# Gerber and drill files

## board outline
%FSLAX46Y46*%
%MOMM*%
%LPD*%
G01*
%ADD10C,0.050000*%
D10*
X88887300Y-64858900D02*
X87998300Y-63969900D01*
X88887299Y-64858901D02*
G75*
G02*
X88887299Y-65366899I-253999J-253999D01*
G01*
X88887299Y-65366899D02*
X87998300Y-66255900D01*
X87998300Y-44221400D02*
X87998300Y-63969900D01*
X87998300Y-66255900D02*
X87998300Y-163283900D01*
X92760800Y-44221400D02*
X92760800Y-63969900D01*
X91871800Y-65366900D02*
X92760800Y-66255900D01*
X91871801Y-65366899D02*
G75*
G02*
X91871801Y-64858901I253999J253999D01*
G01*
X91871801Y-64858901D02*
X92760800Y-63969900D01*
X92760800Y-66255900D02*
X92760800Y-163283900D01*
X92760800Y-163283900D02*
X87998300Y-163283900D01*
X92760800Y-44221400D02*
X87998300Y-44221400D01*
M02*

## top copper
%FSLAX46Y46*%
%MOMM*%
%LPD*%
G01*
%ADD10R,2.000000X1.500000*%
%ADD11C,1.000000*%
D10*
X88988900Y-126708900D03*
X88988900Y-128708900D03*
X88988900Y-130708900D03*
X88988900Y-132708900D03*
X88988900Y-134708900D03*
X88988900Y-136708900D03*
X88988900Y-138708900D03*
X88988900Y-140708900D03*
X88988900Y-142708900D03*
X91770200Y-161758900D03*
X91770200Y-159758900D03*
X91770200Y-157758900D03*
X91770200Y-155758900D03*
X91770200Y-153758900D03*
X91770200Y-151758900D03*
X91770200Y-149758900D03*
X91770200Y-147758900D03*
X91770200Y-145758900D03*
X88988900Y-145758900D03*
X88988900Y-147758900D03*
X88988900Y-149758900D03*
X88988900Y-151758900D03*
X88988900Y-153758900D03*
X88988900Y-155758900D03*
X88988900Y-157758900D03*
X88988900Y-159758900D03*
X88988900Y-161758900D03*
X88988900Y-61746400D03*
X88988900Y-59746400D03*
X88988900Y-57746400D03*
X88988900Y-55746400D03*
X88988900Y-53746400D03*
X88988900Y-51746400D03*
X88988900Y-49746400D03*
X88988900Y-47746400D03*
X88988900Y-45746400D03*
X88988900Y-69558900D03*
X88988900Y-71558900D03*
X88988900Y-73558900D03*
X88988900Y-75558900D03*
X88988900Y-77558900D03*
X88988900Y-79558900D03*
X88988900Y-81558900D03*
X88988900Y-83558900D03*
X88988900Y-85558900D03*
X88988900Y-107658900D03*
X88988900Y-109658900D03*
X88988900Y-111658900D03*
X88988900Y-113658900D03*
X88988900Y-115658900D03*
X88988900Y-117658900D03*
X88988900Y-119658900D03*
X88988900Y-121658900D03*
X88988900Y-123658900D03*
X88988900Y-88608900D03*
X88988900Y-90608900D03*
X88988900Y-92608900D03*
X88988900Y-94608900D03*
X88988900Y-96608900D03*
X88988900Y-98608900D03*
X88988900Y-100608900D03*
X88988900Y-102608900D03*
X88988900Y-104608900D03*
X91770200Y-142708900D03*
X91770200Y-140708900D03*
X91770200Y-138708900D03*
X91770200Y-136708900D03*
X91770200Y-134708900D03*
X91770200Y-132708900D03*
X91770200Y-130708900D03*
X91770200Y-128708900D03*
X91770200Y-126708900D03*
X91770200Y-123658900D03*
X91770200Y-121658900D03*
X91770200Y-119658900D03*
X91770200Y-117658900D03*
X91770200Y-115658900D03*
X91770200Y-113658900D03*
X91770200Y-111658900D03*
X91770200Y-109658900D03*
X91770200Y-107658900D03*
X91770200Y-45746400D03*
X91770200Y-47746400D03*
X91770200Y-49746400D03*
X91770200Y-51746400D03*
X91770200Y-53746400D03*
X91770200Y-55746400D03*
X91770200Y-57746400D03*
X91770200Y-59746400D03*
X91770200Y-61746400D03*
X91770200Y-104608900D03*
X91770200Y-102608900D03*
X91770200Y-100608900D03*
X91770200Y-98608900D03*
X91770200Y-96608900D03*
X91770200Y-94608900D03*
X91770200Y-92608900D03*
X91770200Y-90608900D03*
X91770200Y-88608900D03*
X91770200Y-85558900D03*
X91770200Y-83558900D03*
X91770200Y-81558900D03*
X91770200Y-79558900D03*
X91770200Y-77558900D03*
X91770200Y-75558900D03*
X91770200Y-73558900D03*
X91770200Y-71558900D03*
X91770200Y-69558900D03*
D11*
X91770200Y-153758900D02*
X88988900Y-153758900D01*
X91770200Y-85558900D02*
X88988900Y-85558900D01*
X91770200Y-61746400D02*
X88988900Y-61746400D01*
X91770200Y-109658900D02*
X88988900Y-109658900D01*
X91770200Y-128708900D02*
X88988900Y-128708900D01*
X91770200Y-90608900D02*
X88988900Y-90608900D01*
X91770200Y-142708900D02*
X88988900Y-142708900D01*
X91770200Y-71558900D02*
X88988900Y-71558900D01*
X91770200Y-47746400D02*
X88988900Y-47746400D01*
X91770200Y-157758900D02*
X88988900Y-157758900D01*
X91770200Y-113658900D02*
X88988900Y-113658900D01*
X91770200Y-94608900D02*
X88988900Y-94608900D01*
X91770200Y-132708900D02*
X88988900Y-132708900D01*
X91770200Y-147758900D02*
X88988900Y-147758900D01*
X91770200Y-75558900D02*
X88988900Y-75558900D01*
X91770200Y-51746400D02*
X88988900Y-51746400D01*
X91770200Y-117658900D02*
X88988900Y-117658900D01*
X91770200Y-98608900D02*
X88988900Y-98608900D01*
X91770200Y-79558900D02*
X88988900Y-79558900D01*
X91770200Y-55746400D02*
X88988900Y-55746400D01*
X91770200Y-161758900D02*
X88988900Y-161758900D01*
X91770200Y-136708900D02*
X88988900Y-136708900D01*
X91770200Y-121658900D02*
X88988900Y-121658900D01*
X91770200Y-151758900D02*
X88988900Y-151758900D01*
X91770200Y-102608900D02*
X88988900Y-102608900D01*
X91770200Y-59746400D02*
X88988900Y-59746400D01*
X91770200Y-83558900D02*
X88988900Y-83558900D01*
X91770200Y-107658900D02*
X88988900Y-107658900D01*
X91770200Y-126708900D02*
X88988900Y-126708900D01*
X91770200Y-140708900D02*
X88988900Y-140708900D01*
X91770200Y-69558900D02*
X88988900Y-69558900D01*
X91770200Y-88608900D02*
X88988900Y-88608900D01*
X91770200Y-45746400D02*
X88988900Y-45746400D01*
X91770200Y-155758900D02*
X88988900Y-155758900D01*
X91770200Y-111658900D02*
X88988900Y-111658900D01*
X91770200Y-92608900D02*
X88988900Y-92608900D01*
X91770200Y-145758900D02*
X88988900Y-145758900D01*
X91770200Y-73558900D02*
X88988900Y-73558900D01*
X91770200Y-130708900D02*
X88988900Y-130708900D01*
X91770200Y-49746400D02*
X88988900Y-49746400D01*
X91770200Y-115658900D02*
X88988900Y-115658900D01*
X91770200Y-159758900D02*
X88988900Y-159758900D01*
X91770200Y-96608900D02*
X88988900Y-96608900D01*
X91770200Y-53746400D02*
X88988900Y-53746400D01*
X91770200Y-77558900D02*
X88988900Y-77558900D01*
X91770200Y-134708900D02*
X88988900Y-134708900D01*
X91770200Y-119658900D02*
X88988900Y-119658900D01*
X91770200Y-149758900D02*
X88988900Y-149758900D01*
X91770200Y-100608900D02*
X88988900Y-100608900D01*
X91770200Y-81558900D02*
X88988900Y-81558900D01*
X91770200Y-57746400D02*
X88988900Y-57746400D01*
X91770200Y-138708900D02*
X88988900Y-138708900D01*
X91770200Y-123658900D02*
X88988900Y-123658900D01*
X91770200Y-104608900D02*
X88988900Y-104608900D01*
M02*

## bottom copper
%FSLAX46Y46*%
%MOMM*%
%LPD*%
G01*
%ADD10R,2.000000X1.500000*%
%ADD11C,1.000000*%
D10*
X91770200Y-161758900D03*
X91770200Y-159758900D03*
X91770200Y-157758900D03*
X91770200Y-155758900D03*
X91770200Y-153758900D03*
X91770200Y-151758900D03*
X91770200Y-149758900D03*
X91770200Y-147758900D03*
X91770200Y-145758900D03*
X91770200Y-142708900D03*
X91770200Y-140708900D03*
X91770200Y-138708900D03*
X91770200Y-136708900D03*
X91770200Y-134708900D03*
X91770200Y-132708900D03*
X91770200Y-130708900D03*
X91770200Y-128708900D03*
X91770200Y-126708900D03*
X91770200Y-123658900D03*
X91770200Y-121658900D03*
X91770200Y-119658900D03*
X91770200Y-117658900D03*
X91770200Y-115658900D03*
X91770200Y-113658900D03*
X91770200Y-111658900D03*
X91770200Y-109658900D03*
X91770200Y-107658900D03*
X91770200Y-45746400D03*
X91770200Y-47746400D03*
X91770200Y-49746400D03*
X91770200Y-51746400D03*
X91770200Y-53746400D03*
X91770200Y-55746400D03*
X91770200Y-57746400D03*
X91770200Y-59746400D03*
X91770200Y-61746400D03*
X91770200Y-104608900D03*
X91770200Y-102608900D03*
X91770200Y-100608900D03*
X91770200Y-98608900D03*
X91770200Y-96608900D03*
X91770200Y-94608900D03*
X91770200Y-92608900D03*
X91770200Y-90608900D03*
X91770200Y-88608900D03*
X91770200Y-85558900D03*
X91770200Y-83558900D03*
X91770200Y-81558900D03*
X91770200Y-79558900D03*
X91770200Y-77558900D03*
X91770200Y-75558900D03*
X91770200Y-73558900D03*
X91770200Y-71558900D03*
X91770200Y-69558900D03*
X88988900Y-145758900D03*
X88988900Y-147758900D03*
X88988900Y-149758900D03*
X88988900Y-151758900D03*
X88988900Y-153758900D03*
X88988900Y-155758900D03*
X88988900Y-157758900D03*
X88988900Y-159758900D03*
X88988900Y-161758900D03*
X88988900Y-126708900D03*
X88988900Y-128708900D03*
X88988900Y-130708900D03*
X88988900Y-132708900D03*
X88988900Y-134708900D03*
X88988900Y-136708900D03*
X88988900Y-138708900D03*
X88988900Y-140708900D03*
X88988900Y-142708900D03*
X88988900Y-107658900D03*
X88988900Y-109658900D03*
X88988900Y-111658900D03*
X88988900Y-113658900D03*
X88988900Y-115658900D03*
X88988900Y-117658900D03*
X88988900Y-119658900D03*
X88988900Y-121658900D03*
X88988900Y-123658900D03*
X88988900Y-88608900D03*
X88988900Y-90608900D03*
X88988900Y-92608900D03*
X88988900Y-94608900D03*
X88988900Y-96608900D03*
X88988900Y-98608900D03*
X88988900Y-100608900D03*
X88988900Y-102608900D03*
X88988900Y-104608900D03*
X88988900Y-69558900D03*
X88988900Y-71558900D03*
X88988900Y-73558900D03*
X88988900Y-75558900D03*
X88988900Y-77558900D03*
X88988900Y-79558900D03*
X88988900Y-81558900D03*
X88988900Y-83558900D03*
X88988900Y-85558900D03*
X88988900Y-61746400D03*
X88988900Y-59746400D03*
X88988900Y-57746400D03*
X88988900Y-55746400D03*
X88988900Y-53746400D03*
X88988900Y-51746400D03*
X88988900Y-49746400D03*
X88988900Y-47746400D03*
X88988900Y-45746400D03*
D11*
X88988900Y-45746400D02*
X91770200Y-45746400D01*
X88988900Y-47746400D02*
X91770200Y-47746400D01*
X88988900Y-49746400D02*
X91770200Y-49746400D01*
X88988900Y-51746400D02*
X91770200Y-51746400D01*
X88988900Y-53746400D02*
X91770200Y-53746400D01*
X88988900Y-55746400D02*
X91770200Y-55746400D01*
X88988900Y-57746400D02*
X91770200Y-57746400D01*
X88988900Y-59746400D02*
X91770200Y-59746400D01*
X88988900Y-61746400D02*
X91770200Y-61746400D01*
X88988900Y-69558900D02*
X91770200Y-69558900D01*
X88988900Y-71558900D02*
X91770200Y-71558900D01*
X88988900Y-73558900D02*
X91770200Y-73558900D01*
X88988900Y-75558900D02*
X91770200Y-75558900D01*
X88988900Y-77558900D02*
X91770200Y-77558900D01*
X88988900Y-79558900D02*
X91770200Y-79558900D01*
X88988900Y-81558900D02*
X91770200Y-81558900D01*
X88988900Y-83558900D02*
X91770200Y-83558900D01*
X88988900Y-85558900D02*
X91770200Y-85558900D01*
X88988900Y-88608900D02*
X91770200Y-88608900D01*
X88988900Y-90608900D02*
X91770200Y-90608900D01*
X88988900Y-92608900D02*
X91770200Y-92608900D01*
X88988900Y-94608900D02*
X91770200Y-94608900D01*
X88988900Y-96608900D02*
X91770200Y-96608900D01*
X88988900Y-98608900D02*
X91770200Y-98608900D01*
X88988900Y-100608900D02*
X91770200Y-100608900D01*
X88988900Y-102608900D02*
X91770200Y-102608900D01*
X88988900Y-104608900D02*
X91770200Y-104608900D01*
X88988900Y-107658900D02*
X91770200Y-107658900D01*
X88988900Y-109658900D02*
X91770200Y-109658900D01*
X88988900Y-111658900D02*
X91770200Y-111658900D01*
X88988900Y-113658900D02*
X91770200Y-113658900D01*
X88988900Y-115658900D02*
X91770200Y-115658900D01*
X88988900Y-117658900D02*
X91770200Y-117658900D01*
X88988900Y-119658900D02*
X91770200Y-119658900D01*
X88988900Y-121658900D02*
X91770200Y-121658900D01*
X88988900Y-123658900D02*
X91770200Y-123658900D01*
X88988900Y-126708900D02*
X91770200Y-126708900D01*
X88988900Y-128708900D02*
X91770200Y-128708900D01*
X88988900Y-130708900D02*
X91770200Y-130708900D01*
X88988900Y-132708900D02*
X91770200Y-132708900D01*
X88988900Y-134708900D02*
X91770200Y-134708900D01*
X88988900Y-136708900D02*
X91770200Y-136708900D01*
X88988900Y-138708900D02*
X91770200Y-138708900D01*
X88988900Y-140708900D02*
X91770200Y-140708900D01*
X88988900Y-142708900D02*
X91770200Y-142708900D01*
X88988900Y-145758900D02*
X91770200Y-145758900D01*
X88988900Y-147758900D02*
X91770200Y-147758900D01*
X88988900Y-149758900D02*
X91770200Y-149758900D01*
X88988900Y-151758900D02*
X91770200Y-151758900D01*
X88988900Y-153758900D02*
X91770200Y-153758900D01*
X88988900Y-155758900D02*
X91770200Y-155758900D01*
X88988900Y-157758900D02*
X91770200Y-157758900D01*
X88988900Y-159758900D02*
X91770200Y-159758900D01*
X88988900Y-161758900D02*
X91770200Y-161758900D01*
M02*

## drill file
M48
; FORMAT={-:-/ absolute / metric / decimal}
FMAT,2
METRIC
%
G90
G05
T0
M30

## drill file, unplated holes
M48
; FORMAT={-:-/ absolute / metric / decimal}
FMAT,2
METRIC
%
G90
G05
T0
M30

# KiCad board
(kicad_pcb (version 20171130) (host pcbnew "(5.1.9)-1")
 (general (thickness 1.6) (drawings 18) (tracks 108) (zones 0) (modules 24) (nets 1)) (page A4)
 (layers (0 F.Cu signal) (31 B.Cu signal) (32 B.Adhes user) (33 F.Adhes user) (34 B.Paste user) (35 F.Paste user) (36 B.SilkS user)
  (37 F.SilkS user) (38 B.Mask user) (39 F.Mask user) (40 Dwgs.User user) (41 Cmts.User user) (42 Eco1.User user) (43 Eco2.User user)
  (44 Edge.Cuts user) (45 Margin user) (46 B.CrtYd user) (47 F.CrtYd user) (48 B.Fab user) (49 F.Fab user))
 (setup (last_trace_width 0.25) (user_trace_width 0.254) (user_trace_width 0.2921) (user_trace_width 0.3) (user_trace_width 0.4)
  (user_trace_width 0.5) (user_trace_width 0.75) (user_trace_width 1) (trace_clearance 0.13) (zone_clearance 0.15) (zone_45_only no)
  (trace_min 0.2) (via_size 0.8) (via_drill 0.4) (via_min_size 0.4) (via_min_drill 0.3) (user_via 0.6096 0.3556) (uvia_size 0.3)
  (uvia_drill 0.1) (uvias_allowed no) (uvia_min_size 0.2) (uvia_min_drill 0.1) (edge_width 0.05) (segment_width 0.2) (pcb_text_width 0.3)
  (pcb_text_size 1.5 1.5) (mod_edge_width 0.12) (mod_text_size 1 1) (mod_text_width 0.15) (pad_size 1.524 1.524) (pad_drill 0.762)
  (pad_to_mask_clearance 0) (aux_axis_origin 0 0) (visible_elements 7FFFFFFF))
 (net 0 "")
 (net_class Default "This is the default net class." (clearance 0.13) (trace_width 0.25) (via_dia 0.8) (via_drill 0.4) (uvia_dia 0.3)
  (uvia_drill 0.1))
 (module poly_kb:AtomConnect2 (layer F.Cu) (at 88.9889 134.7089 270)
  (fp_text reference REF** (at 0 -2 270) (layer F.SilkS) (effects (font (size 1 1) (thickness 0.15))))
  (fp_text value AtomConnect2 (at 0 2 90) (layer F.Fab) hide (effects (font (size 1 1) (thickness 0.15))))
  (pad 1 smd rect (at -8 0 270) (size 1.5 2) (layers F.Cu F.Mask) (zone_connect 0))
  (pad 2 smd rect (at -6 0 270) (size 1.5 2) (layers F.Cu F.Mask) (zone_connect 0))
  (pad 3 smd rect (at -4 0 270) (size 1.5 2) (layers F.Cu F.Mask) (zone_connect 0))
  (pad 4 smd rect (at -2 0 270) (size 1.5 2) (layers F.Cu F.Mask) (zone_connect 0))
  (pad 5 smd rect (at 0 0 270) (size 1.5 2) (layers F.Cu F.Mask) (zone_connect 0))
  (pad 6 smd rect (at 2 0 270) (size 1.5 2) (layers F.Cu F.Mask) (zone_connect 0))
  (pad 7 smd rect (at 4 0 270) (size 1.5 2) (layers F.Cu F.Mask) (zone_connect 0))
  (pad 8 smd rect (at 6 0 270) (size 1.5 2) (layers F.Cu F.Mask) (zone_connect 0))
  (pad 9 smd rect (at 8 0 270) (size 1.5 2) (layers F.Cu F.Mask) (zone_connect 0)))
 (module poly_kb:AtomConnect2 (layer F.Cu) (at 91.7702 153.7589 270)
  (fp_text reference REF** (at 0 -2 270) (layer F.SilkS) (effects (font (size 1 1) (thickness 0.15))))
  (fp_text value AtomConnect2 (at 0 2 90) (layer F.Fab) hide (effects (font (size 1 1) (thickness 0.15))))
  (pad 9 smd rect (at 8 0 270) (size 1.5 2) (layers F.Cu F.Mask) (zone_connect 0))
  (pad 8 smd rect (at 6 0 270) (size 1.5 2) (layers F.Cu F.Mask) (zone_connect 0))
  (pad 7 smd rect (at 4 0 270) (size 1.5 2) (layers F.Cu F.Mask) (zone_connect 0))
  (pad 6 smd rect (at 2 0 270) (size 1.5 2) (layers F.Cu F.Mask) (zone_connect 0))
  (pad 5 smd rect (at 0 0 270) (size 1.5 2) (layers F.Cu F.Mask) (zone_connect 0))
  (pad 4 smd rect (at -2 0 270) (size 1.5 2) (layers F.Cu F.Mask) (zone_connect 0))
  (pad 3 smd rect (at -4 0 270) (size 1.5 2) (layers F.Cu F.Mask) (zone_connect 0))
  (pad 2 smd rect (at -6 0 270) (size 1.5 2) (layers F.Cu F.Mask) (zone_connect 0))
  (pad 1 smd rect (at -8 0 270) (size 1.5 2) (layers F.Cu F.Mask) (zone_connect 0)))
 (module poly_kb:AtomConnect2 (layer F.Cu) (at 88.9889 153.7589 270)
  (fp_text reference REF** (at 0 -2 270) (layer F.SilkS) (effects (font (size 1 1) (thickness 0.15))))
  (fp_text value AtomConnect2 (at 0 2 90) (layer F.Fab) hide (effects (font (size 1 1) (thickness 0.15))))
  (pad 1 smd rect (at -8 0 270) (size 1.5 2) (layers F.Cu F.Mask) (zone_connect 0))
  (pad 2 smd rect (at -6 0 270) (size 1.5 2) (layers F.Cu F.Mask) (zone_connect 0))
  (pad 3 smd rect (at -4 0 270) (size 1.5 2) (layers F.Cu F.Mask) (zone_connect 0))
  (pad 4 smd rect (at -2 0 270) (size 1.5 2) (layers F.Cu F.Mask) (zone_connect 0))
  (pad 5 smd rect (at 0 0 270) (size 1.5 2) (layers F.Cu F.Mask) (zone_connect 0))
  (pad 6 smd rect (at 2 0 270) (size 1.5 2) (layers F.Cu F.Mask) (zone_connect 0))
  (pad 7 smd rect (at 4 0 270) (size 1.5 2) (layers F.Cu F.Mask) (zone_connect 0))
  (pad 8 smd rect (at 6 0 270) (size 1.5 2) (layers F.Cu F.Mask) (zone_connect 0))
  (pad 9 smd rect (at 8 0 270) (size 1.5 2) (layers F.Cu F.Mask) (zone_connect 0)))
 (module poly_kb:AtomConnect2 (layer F.Cu) (at 88.9889 53.7464 270)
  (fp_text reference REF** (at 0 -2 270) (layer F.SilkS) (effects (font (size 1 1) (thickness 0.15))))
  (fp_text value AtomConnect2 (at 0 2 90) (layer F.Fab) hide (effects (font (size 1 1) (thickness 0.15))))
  (pad 9 smd rect (at 8 0 270) (size 1.5 2) (layers F.Cu F.Mask) (zone_connect 0))
  (pad 8 smd rect (at 6 0 270) (size 1.5 2) (layers F.Cu F.Mask) (zone_connect 0))
  (pad 7 smd rect (at 4 0 270) (size 1.5 2) (layers F.Cu F.Mask) (zone_connect 0))
  (pad 6 smd rect (at 2 0 270) (size 1.5 2) (layers F.Cu F.Mask) (zone_connect 0))
  (pad 5 smd rect (at 0 0 270) (size 1.5 2) (layers F.Cu F.Mask) (zone_connect 0))
  (pad 4 smd rect (at -2 0 270) (size 1.5 2) (layers F.Cu F.Mask) (zone_connect 0))
  (pad 3 smd rect (at -4 0 270) (size 1.5 2) (layers F.Cu F.Mask) (zone_connect 0))
  (pad 2 smd rect (at -6 0 270) (size 1.5 2) (layers F.Cu F.Mask) (zone_connect 0))
  (pad 1 smd rect (at -8 0 270) (size 1.5 2) (layers F.Cu F.Mask) (zone_connect 0)))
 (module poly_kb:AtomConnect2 (layer F.Cu) (at 88.9889 77.5589 270)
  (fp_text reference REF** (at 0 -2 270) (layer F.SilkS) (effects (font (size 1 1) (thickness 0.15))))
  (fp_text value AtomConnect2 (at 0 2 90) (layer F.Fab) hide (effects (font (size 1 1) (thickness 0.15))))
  (pad 1 smd rect (at -8 0 270) (size 1.5 2) (layers F.Cu F.Mask) (zone_connect 0))
  (pad 2 smd rect (at -6 0 270) (size 1.5 2) (layers F.Cu F.Mask) (zone_connect 0))
  (pad 3 smd rect (at -4 0 270) (size 1.5 2) (layers F.Cu F.Mask) (zone_connect 0))
  (pad 4 smd rect (at -2 0 270) (size 1.5 2) (layers F.Cu F.Mask) (zone_connect 0))
  (pad 5 smd rect (at 0 0 270) (size 1.5 2) (layers F.Cu F.Mask) (zone_connect 0))
  (pad 6 smd rect (at 2 0 270) (size 1.5 2) (layers F.Cu F.Mask) (zone_connect 0))
  (pad 7 smd rect (at 4 0 270) (size 1.5 2) (layers F.Cu F.Mask) (zone_connect 0))
  (pad 8 smd rect (at 6 0 270) (size 1.5 2) (layers F.Cu F.Mask) (zone_connect 0))
  (pad 9 smd rect (at 8 0 270) (size 1.5 2) (layers F.Cu F.Mask) (zone_connect 0)))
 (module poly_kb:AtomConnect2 (layer F.Cu) (at 88.9889 115.6589 270)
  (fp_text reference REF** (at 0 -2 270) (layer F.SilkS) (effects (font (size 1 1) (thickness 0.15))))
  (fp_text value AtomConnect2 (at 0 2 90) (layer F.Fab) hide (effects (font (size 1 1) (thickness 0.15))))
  (pad 1 smd rect (at -8 0 270) (size 1.5 2) (layers F.Cu F.Mask) (zone_connect 0))
  (pad 2 smd rect (at -6 0 270) (size 1.5 2) (layers F.Cu F.Mask) (zone_connect 0))
  (pad 3 smd rect (at -4 0 270) (size 1.5 2) (layers F.Cu F.Mask) (zone_connect 0))
  (pad 4 smd rect (at -2 0 270) (size 1.5 2) (layers F.Cu F.Mask) (zone_connect 0))
  (pad 5 smd rect (at 0 0 270) (size 1.5 2) (layers F.Cu F.Mask) (zone_connect 0))
  (pad 6 smd rect (at 2 0 270) (size 1.5 2) (layers F.Cu F.Mask) (zone_connect 0))
  (pad 7 smd rect (at 4 0 270) (size 1.5 2) (layers F.Cu F.Mask) (zone_connect 0))
  (pad 8 smd rect (at 6 0 270) (size 1.5 2) (layers F.Cu F.Mask) (zone_connect 0))
  (pad 9 smd rect (at 8 0 270) (size 1.5 2) (layers F.Cu F.Mask) (zone_connect 0)))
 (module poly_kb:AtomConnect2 (layer F.Cu) (at 88.9889 96.6089 270)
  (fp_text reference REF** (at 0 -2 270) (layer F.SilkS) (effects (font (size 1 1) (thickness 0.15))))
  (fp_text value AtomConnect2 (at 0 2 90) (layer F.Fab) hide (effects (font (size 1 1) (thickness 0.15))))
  (pad 1 smd rect (at -8 0 270) (size 1.5 2) (layers F.Cu F.Mask) (zone_connect 0))
  (pad 2 smd rect (at -6 0 270) (size 1.5 2) (layers F.Cu F.Mask) (zone_connect 0))
  (pad 3 smd rect (at -4 0 270) (size 1.5 2) (layers F.Cu F.Mask) (zone_connect 0))
  (pad 4 smd rect (at -2 0 270) (size 1.5 2) (layers F.Cu F.Mask) (zone_connect 0))
  (pad 5 smd rect (at 0 0 270) (size 1.5 2) (layers F.Cu F.Mask) (zone_connect 0))
  (pad 6 smd rect (at 2 0 270) (size 1.5 2) (layers F.Cu F.Mask) (zone_connect 0))
  (pad 7 smd rect (at 4 0 270) (size 1.5 2) (layers F.Cu F.Mask) (zone_connect 0))
  (pad 8 smd rect (at 6 0 270) (size 1.5 2) (layers F.Cu F.Mask) (zone_connect 0))
  (pad 9 smd rect (at 8 0 270) (size 1.5 2) (layers F.Cu F.Mask) (zone_connect 0)))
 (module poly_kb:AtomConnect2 (layer F.Cu) (at 91.7702 134.7089 270)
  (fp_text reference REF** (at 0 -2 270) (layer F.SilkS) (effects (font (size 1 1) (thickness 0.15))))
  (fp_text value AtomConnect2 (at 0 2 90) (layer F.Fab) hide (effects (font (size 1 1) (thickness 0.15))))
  (pad 9 smd rect (at 8 0 270) (size 1.5 2) (layers F.Cu F.Mask) (zone_connect 0))
  (pad 8 smd rect (at 6 0 270) (size 1.5 2) (layers F.Cu F.Mask) (zone_connect 0))
  (pad 7 smd rect (at 4 0 270) (size 1.5 2) (layers F.Cu F.Mask) (zone_connect 0))
  (pad 6 smd rect (at 2 0 270) (size 1.5 2) (layers F.Cu F.Mask) (zone_connect 0))
  (pad 5 smd rect (at 0 0 270) (size 1.5 2) (layers F.Cu F.Mask) (zone_connect 0))
  (pad 4 smd rect (at -2 0 270) (size 1.5 2) (layers F.Cu F.Mask) (zone_connect 0))
  (pad 3 smd rect (at -4 0 270) (size 1.5 2) (layers F.Cu F.Mask) (zone_connect 0))
  (pad 2 smd rect (at -6 0 270) (size 1.5 2) (layers F.Cu F.Mask) (zone_connect 0))
  (pad 1 smd rect (at -8 0 270) (size 1.5 2) (layers F.Cu F.Mask) (zone_connect 0)))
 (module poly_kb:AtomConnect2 (layer F.Cu) (at 91.7702 115.6589 270)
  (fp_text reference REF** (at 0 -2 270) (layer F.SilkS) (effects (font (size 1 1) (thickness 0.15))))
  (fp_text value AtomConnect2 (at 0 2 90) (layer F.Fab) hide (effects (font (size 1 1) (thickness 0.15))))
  (pad 9 smd rect (at 8 0 270) (size 1.5 2) (layers F.Cu F.Mask) (zone_connect 0))
  (pad 8 smd rect (at 6 0 270) (size 1.5 2) (layers F.Cu F.Mask) (zone_connect 0))
  (pad 7 smd rect (at 4 0 270) (size 1.5 2) (layers F.Cu F.Mask) (zone_connect 0))
  (pad 6 smd rect (at 2 0 270) (size 1.5 2) (layers F.Cu F.Mask) (zone_connect 0))
  (pad 5 smd rect (at 0 0 270) (size 1.5 2) (layers F.Cu F.Mask) (zone_connect 0))
  (pad 4 smd rect (at -2 0 270) (size 1.5 2) (layers F.Cu F.Mask) (zone_connect 0))
  (pad 3 smd rect (at -4 0 270) (size 1.5 2) (layers F.Cu F.Mask) (zone_connect 0))
  (pad 2 smd rect (at -6 0 270) (size 1.5 2) (layers F.Cu F.Mask) (zone_connect 0))
  (pad 1 smd rect (at -8 0 270) (size 1.5 2) (layers F.Cu F.Mask) (zone_connect 0)))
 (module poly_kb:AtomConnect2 (layer F.Cu) (at 91.7702 53.7464 270)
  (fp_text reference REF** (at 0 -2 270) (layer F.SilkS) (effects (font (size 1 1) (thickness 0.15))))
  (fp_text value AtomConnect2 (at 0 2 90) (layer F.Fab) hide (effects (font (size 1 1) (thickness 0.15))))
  (pad 1 smd rect (at -8 0 270) (size 1.5 2) (layers F.Cu F.Mask) (zone_connect 0))
  (pad 2 smd rect (at -6 0 270) (size 1.5 2) (layers F.Cu F.Mask) (zone_connect 0))
  (pad 3 smd rect (at -4 0 270) (size 1.5 2) (layers F.Cu F.Mask) (zone_connect 0))
  (pad 4 smd rect (at -2 0 270) (size 1.5 2) (layers F.Cu F.Mask) (zone_connect 0))
  (pad 5 smd rect (at 0 0 270) (size 1.5 2) (layers F.Cu F.Mask) (zone_connect 0))
  (pad 6 smd rect (at 2 0 270) (size 1.5 2) (layers F.Cu F.Mask) (zone_connect 0))
  (pad 7 smd rect (at 4 0 270) (size 1.5 2) (layers F.Cu F.Mask) (zone_connect 0))
  (pad 8 smd rect (at 6 0 270) (size 1.5 2) (layers F.Cu F.Mask) (zone_connect 0))
  (pad 9 smd rect (at 8 0 270) (size 1.5 2) (layers F.Cu F.Mask) (zone_connect 0)))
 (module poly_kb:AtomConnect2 (layer F.Cu) (at 91.7702 96.6089 270)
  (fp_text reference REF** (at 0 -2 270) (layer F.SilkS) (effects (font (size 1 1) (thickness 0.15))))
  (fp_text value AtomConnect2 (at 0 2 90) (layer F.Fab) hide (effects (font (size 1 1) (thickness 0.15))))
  (pad 9 smd rect (at 8 0 270) (size 1.5 2) (layers F.Cu F.Mask) (zone_connect 0))
  (pad 8 smd rect (at 6 0 270) (size 1.5 2) (layers F.Cu F.Mask) (zone_connect 0))
  (pad 7 smd rect (at 4 0 270) (size 1.5 2) (layers F.Cu F.Mask) (zone_connect 0))
  (pad 6 smd rect (at 2 0 270) (size 1.5 2) (layers F.Cu F.Mask) (zone_connect 0))
  (pad 5 smd rect (at 0 0 270) (size 1.5 2) (layers F.Cu F.Mask) (zone_connect 0))
  (pad 4 smd rect (at -2 0 270) (size 1.5 2) (layers F.Cu F.Mask) (zone_connect 0))
  (pad 3 smd rect (at -4 0 270) (size 1.5 2) (layers F.Cu F.Mask) (zone_connect 0))
  (pad 2 smd rect (at -6 0 270) (size 1.5 2) (layers F.Cu F.Mask) (zone_connect 0))
  (pad 1 smd rect (at -8 0 270) (size 1.5 2) (layers F.Cu F.Mask) (zone_connect 0)))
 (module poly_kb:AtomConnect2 (layer F.Cu) (at 91.7702 77.5589 270)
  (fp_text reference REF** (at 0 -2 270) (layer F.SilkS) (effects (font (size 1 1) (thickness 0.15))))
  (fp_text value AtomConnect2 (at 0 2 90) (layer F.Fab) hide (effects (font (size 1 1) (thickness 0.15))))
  (pad 9 smd rect (at 8 0 270) (size 1.5 2) (layers F.Cu F.Mask) (zone_connect 0))
  (pad 8 smd rect (at 6 0 270) (size 1.5 2) (layers F.Cu F.Mask) (zone_connect 0))
  (pad 7 smd rect (at 4 0 270) (size 1.5 2) (layers F.Cu F.Mask) (zone_connect 0))
  (pad 6 smd rect (at 2 0 270) (size 1.5 2) (layers F.Cu F.Mask) (zone_connect 0))
  (pad 5 smd rect (at 0 0 270) (size 1.5 2) (layers F.Cu F.Mask) (zone_connect 0))
  (pad 4 smd rect (at -2 0 270) (size 1.5 2) (layers F.Cu F.Mask) (zone_connect 0))
  (pad 3 smd rect (at -4 0 270) (size 1.5 2) (layers F.Cu F.Mask) (zone_connect 0))
  (pad 2 smd rect (at -6 0 270) (size 1.5 2) (layers F.Cu F.Mask) (zone_connect 0))
  (pad 1 smd rect (at -8 0 270) (size 1.5 2) (layers F.Cu F.Mask) (zone_connect 0)))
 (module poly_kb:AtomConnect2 (layer B.Cu) (at 91.7702 153.7589 270)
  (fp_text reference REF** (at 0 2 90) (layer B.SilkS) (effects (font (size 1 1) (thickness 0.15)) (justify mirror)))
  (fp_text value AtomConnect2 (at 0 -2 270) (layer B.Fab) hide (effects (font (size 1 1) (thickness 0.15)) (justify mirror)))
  (pad 9 smd rect (at 8 0 270) (size 1.5 2) (layers B.Cu B.Mask) (zone_connect 0))
  (pad 8 smd rect (at 6 0 270) (size 1.5 2) (layers B.Cu B.Mask) (zone_connect 0))
  (pad 7 smd rect (at 4 0 270) (size 1.5 2) (layers B.Cu B.Mask) (zone_connect 0))
  (pad 6 smd rect (at 2 0 270) (size 1.5 2) (layers B.Cu B.Mask) (zone_connect 0))
  (pad 5 smd rect (at 0 0 270) (size 1.5 2) (layers B.Cu B.Mask) (zone_connect 0))
  (pad 4 smd rect (at -2 0 270) (size 1.5 2) (layers B.Cu B.Mask) (zone_connect 0))
  (pad 3 smd rect (at -4 0 270) (size 1.5 2) (layers B.Cu B.Mask) (zone_connect 0))
  (pad 2 smd rect (at -6 0 270) (size 1.5 2) (layers B.Cu B.Mask) (zone_connect 0))
  (pad 1 smd rect (at -8 0 270) (size 1.5 2) (layers B.Cu B.Mask) (zone_connect 0)))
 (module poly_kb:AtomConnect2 (layer B.Cu) (at 91.7702 134.7089 270)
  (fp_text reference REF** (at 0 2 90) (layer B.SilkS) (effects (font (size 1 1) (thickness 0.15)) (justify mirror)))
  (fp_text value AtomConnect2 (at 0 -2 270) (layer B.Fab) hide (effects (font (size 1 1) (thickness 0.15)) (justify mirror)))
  (pad 9 smd rect (at 8 0 270) (size 1.5 2) (layers B.Cu B.Mask) (zone_connect 0))
  (pad 8 smd rect (at 6 0 270) (size 1.5 2) (layers B.Cu B.Mask) (zone_connect 0))
  (pad 7 smd rect (at 4 0 270) (size 1.5 2) (layers B.Cu B.Mask) (zone_connect 0))
  (pad 6 smd rect (at 2 0 270) (size 1.5 2) (layers B.Cu B.Mask) (zone_connect 0))
  (pad 5 smd rect (at 0 0 270) (size 1.5 2) (layers B.Cu B.Mask) (zone_connect 0))
  (pad 4 smd rect (at -2 0 270) (size 1.5 2) (layers B.Cu B.Mask) (zone_connect 0))
  (pad 3 smd rect (at -4 0 270) (size 1.5 2) (layers B.Cu B.Mask) (zone_connect 0))
  (pad 2 smd rect (at -6 0 270) (size 1.5 2) (layers B.Cu B.Mask) (zone_connect 0))
  (pad 1 smd rect (at -8 0 270) (size 1.5 2) (layers B.Cu B.Mask) (zone_connect 0)))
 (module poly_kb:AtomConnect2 (layer B.Cu) (at 91.7702 115.6589 270)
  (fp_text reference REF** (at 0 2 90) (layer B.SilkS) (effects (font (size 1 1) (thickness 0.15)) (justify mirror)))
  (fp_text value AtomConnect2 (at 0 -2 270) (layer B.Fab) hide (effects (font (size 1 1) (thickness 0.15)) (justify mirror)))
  (pad 9 smd rect (at 8 0 270) (size 1.5 2) (layers B.Cu B.Mask) (zone_connect 0))
  (pad 8 smd rect (at 6 0 270) (size 1.5 2) (layers B.Cu B.Mask) (zone_connect 0))
  (pad 7 smd rect (at 4 0 270) (size 1.5 2) (layers B.Cu B.Mask) (zone_connect 0))
  (pad 6 smd rect (at 2 0 270) (size 1.5 2) (layers B.Cu B.Mask) (zone_connect 0))
  (pad 5 smd rect (at 0 0 270) (size 1.5 2) (layers B.Cu B.Mask) (zone_connect 0))
  (pad 4 smd rect (at -2 0 270) (size 1.5 2) (layers B.Cu B.Mask) (zone_connect 0))
  (pad 3 smd rect (at -4 0 270) (size 1.5 2) (layers B.Cu B.Mask) (zone_connect 0))
  (pad 2 smd rect (at -6 0 270) (size 1.5 2) (layers B.Cu B.Mask) (zone_connect 0))
  (pad 1 smd rect (at -8 0 270) (size 1.5 2) (layers B.Cu B.Mask) (zone_connect 0)))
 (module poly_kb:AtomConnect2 (layer B.Cu) (at 91.7702 53.7464 270)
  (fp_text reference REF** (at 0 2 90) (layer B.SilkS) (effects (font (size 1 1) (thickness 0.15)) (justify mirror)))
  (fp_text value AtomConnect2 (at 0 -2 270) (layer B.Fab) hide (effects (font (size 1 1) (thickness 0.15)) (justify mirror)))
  (pad 1 smd rect (at -8 0 270) (size 1.5 2) (layers B.Cu B.Mask) (zone_connect 0))
  (pad 2 smd rect (at -6 0 270) (size 1.5 2) (layers B.Cu B.Mask) (zone_connect 0))
  (pad 3 smd rect (at -4 0 270) (size 1.5 2) (layers B.Cu B.Mask) (zone_connect 0))
  (pad 4 smd rect (at -2 0 270) (size 1.5 2) (layers B.Cu B.Mask) (zone_connect 0))
  (pad 5 smd rect (at 0 0 270) (size 1.5 2) (layers B.Cu B.Mask) (zone_connect 0))
  (pad 6 smd rect (at 2 0 270) (size 1.5 2) (layers B.Cu B.Mask) (zone_connect 0))
  (pad 7 smd rect (at 4 0 270) (size 1.5 2) (layers B.Cu B.Mask) (zone_connect 0))
  (pad 8 smd rect (at 6 0 270) (size 1.5 2) (layers B.Cu B.Mask) (zone_connect 0))
  (pad 9 smd rect (at 8 0 270) (size 1.5 2) (layers B.Cu B.Mask) (zone_connect 0)))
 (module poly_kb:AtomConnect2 (layer B.Cu) (at 91.7702 96.6089 270)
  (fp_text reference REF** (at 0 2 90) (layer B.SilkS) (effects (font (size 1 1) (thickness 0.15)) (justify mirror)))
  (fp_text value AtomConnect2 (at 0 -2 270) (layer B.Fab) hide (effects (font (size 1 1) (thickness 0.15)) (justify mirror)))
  (pad 9 smd rect (at 8 0 270) (size 1.5 2) (layers B.Cu B.Mask) (zone_connect 0))
  (pad 8 smd rect (at 6 0 270) (size 1.5 2) (layers B.Cu B.Mask) (zone_connect 0))
  (pad 7 smd rect (at 4 0 270) (size 1.5 2) (layers B.Cu B.Mask) (zone_connect 0))
  (pad 6 smd rect (at 2 0 270) (size 1.5 2) (layers B.Cu B.Mask) (zone_connect 0))
  (pad 5 smd rect (at 0 0 270) (size 1.5 2) (layers B.Cu B.Mask) (zone_connect 0))
  (pad 4 smd rect (at -2 0 270) (size 1.5 2) (layers B.Cu B.Mask) (zone_connect 0))
  (pad 3 smd rect (at -4 0 270) (size 1.5 2) (layers B.Cu B.Mask) (zone_connect 0))
  (pad 2 smd rect (at -6 0 270) (size 1.5 2) (layers B.Cu B.Mask) (zone_connect 0))
  (pad 1 smd rect (at -8 0 270) (size 1.5 2) (layers B.Cu B.Mask) (zone_connect 0)))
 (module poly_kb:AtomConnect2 (layer B.Cu) (at 91.7702 77.5589 270)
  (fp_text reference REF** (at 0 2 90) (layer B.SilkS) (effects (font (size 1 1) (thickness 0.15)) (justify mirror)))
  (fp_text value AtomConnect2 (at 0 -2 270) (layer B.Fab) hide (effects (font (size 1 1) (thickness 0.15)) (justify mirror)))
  (pad 9 smd rect (at 8 0 270) (size 1.5 2) (layers B.Cu B.Mask) (zone_connect 0))
  (pad 8 smd rect (at 6 0 270) (size 1.5 2) (layers B.Cu B.Mask) (zone_connect 0))
  (pad 7 smd rect (at 4 0 270) (size 1.5 2) (layers B.Cu B.Mask) (zone_connect 0))
  (pad 6 smd rect (at 2 0 270) (size 1.5 2) (layers B.Cu B.Mask) (zone_connect 0))
  (pad 5 smd rect (at 0 0 270) (size 1.5 2) (layers B.Cu B.Mask) (zone_connect 0))
  (pad 4 smd rect (at -2 0 270) (size 1.5 2) (layers B.Cu B.Mask) (zone_connect 0))
  (pad 3 smd rect (at -4 0 270) (size 1.5 2) (layers B.Cu B.Mask) (zone_connect 0))
  (pad 2 smd rect (at -6 0 270) (size 1.5 2) (layers B.Cu B.Mask) (zone_connect 0))
  (pad 1 smd rect (at -8 0 270) (size 1.5 2) (layers B.Cu B.Mask) (zone_connect 0)))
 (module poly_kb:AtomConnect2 (layer B.Cu) (at 88.9889 153.7589 270)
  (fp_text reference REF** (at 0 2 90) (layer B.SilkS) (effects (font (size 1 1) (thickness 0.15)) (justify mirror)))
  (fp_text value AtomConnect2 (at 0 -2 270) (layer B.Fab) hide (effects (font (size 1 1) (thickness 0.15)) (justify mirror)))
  (pad 1 smd rect (at -8 0 270) (size 1.5 2) (layers B.Cu B.Mask) (zone_connect 0))
  (pad 2 smd rect (at -6 0 270) (size 1.5 2) (layers B.Cu B.Mask) (zone_connect 0))
  (pad 3 smd rect (at -4 0 270) (size 1.5 2) (layers B.Cu B.Mask) (zone_connect 0))
  (pad 4 smd rect (at -2 0 270) (size 1.5 2) (layers B.Cu B.Mask) (zone_connect 0))
  (pad 5 smd rect (at 0 0 270) (size 1.5 2) (layers B.Cu B.Mask) (zone_connect 0))
  (pad 6 smd rect (at 2 0 270) (size 1.5 2) (layers B.Cu B.Mask) (zone_connect 0))
  (pad 7 smd rect (at 4 0 270) (size 1.5 2) (layers B.Cu B.Mask) (zone_connect 0))
  (pad 8 smd rect (at 6 0 270) (size 1.5 2) (layers B.Cu B.Mask) (zone_connect 0))
  (pad 9 smd rect (at 8 0 270) (size 1.5 2) (layers B.Cu B.Mask) (zone_connect 0)))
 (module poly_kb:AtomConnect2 (layer B.Cu) (at 88.9889 134.7089 270)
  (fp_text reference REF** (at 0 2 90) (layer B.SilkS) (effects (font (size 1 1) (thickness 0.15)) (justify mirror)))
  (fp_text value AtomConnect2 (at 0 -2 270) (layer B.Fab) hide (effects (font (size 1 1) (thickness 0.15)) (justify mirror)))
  (pad 1 smd rect (at -8 0 270) (size 1.5 2) (layers B.Cu B.Mask) (zone_connect 0))
  (pad 2 smd rect (at -6 0 270) (size 1.5 2) (layers B.Cu B.Mask) (zone_connect 0))
  (pad 3 smd rect (at -4 0 270) (size 1.5 2) (layers B.Cu B.Mask) (zone_connect 0))
  (pad 4 smd rect (at -2 0 270) (size 1.5 2) (layers B.Cu B.Mask) (zone_connect 0))
  (pad 5 smd rect (at 0 0 270) (size 1.5 2) (layers B.Cu B.Mask) (zone_connect 0))
  (pad 6 smd rect (at 2 0 270) (size 1.5 2) (layers B.Cu B.Mask) (zone_connect 0))
  (pad 7 smd rect (at 4 0 270) (size 1.5 2) (layers B.Cu B.Mask) (zone_connect 0))
  (pad 8 smd rect (at 6 0 270) (size 1.5 2) (layers B.Cu B.Mask) (zone_connect 0))
  (pad 9 smd rect (at 8 0 270) (size 1.5 2) (layers B.Cu B.Mask) (zone_connect 0)))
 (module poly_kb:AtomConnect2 (layer B.Cu) (at 88.9889 115.6589 270)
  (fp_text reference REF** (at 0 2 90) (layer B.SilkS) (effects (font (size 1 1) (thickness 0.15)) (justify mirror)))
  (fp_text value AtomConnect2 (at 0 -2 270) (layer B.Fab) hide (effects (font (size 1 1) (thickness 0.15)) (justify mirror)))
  (pad 1 smd rect (at -8 0 270) (size 1.5 2) (layers B.Cu B.Mask) (zone_connect 0))
  (pad 2 smd rect (at -6 0 270) (size 1.5 2) (layers B.Cu B.Mask) (zone_connect 0))
  (pad 3 smd rect (at -4 0 270) (size 1.5 2) (layers B.Cu B.Mask) (zone_connect 0))
  (pad 4 smd rect (at -2 0 270) (size 1.5 2) (layers B.Cu B.Mask) (zone_connect 0))
  (pad 5 smd rect (at 0 0 270) (size 1.5 2) (layers B.Cu B.Mask) (zone_connect 0))
  (pad 6 smd rect (at 2 0 270) (size 1.5 2) (layers B.Cu B.Mask) (zone_connect 0))
  (pad 7 smd rect (at 4 0 270) (size 1.5 2) (layers B.Cu B.Mask) (zone_connect 0))
  (pad 8 smd rect (at 6 0 270) (size 1.5 2) (layers B.Cu B.Mask) (zone_connect 0))
  (pad 9 smd rect (at 8 0 270) (size 1.5 2) (layers B.Cu B.Mask) (zone_connect 0)))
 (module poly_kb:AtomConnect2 (layer B.Cu) (at 88.9889 96.6089 270)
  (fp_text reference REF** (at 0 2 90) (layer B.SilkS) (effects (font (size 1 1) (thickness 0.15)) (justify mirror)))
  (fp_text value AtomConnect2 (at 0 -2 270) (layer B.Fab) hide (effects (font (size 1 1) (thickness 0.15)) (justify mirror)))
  (pad 1 smd rect (at -8 0 270) (size 1.5 2) (layers B.Cu B.Mask) (zone_connect 0))
  (pad 2 smd rect (at -6 0 270) (size 1.5 2) (layers B.Cu B.Mask) (zone_connect 0))
  (pad 3 smd rect (at -4 0 270) (size 1.5 2) (layers B.Cu B.Mask) (zone_connect 0))
  (pad 4 smd rect (at -2 0 270) (size 1.5 2) (layers B.Cu B.Mask) (zone_connect 0))
  (pad 5 smd rect (at 0 0 270) (size 1.5 2) (layers B.Cu B.Mask) (zone_connect 0))
  (pad 6 smd rect (at 2 0 270) (size 1.5 2) (layers B.Cu B.Mask) (zone_connect 0))
  (pad 7 smd rect (at 4 0 270) (size 1.5 2) (layers B.Cu B.Mask) (zone_connect 0))
  (pad 8 smd rect (at 6 0 270) (size 1.5 2) (layers B.Cu B.Mask) (zone_connect 0))
  (pad 9 smd rect (at 8 0 270) (size 1.5 2) (layers B.Cu B.Mask) (zone_connect 0)))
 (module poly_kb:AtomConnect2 (layer B.Cu) (at 88.9889 77.5589 270)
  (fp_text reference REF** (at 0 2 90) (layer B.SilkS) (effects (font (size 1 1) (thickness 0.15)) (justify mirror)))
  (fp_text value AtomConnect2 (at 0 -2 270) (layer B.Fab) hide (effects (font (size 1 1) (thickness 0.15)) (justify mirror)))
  (pad 1 smd rect (at -8 0 270) (size 1.5 2) (layers B.Cu B.Mask) (zone_connect 0))
  (pad 2 smd rect (at -6 0 270) (size 1.5 2) (layers B.Cu B.Mask) (zone_connect 0))
  (pad 3 smd rect (at -4 0 270) (size 1.5 2) (layers B.Cu B.Mask) (zone_connect 0))
  (pad 4 smd rect (at -2 0 270) (size 1.5 2) (layers B.Cu B.Mask) (zone_connect 0))
  (pad 5 smd rect (at 0 0 270) (size 1.5 2) (layers B.Cu B.Mask) (zone_connect 0))
  (pad 6 smd rect (at 2 0 270) (size 1.5 2) (layers B.Cu B.Mask) (zone_connect 0))
  (pad 7 smd rect (at 4 0 270) (size 1.5 2) (layers B.Cu B.Mask) (zone_connect 0))
  (pad 8 smd rect (at 6 0 270) (size 1.5 2) (layers B.Cu B.Mask) (zone_connect 0))
  (pad 9 smd rect (at 8 0 270) (size 1.5 2) (layers B.Cu B.Mask) (zone_connect 0)))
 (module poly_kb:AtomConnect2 (layer B.Cu) (at 88.9889 53.7464 270)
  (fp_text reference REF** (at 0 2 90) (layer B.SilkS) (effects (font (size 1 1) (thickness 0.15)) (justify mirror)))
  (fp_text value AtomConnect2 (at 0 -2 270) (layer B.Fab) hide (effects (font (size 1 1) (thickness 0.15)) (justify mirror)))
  (pad 9 smd rect (at 8 0 270) (size 1.5 2) (layers B.Cu B.Mask) (zone_connect 0))
  (pad 8 smd rect (at 6 0 270) (size 1.5 2) (layers B.Cu B.Mask) (zone_connect 0))
  (pad 7 smd rect (at 4 0 270) (size 1.5 2) (layers B.Cu B.Mask) (zone_connect 0))
  (pad 6 smd rect (at 2 0 270) (size 1.5 2) (layers B.Cu B.Mask) (zone_connect 0))
  (pad 5 smd rect (at 0 0 270) (size 1.5 2) (layers B.Cu B.Mask) (zone_connect 0))
  (pad 4 smd rect (at -2 0 270) (size 1.5 2) (layers B.Cu B.Mask) (zone_connect 0))
  (pad 3 smd rect (at -4 0 270) (size 1.5 2) (layers B.Cu B.Mask) (zone_connect 0))
  (pad 2 smd rect (at -6 0 270) (size 1.5 2) (layers B.Cu B.Mask) (zone_connect 0))
  (pad 1 smd rect (at -8 0 270) (size 1.5 2) (layers B.Cu B.Mask) (zone_connect 0)))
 (gr_line (start 88.8873 64.8589) (end 87.9983 63.9699) (layer Edge.Cuts) (width 0.05))
 (gr_arc (start 88.6333 65.1129) (end 88.887299 65.366899) (angle -90) (layer Edge.Cuts) (width 0.05))
 (gr_line (start 88.887299 65.366899) (end 87.9983 66.2559) (layer Edge.Cuts) (width 0.05))
 (gr_line (start 87.9983 44.2214) (end 87.9983 63.9699) (layer Edge.Cuts) (width 0.05))
 (gr_line (start 87.9983 66.2559) (end 87.9983 163.2839) (layer Edge.Cuts) (width 0.05))
 (gr_line (start 92.7608 44.2214) (end 92.7608 63.9699) (layer Edge.Cuts) (width 0.05))
 (gr_line (start 91.8718 65.3669) (end 92.7608 66.2559) (layer Edge.Cuts) (width 0.05))
 (gr_arc (start 92.1258 65.1129) (end 91.871801 64.858901) (angle -90) (layer Edge.Cuts) (width 0.05))
 (gr_line (start 91.871801 64.858901) (end 92.7608 63.9699) (layer Edge.Cuts) (width 0.05))
 (gr_line (start 92.7608 66.2559) (end 92.7608 163.2839) (layer Edge.Cuts) (width 0.05))
 (gr_line (start 92.7608 163.2839) (end 87.9983 163.2839) (layer Edge.Cuts) (width 0.05))
 (gr_line (start 92.7608 44.2214) (end 87.9983 44.2214) (layer Edge.Cuts) (width 0.05))
 (segment (start 88.9889 45.7464) (end 91.7702 45.7464) (width 1) (layer B.Cu) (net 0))
 (segment (start 88.9889 47.7464) (end 91.7702 47.7464) (width 1) (layer B.Cu) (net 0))
 (segment (start 88.9889 49.7464) (end 91.7702 49.7464) (width 1) (layer B.Cu) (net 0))
 (segment (start 88.9889 51.7464) (end 91.7702 51.7464) (width 1) (layer B.Cu) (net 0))
 (segment (start 88.9889 53.7464) (end 91.7702 53.7464) (width 1) (layer B.Cu) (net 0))
 (segment (start 88.9889 55.7464) (end 91.7702 55.7464) (width 1) (layer B.Cu) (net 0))
 (segment (start 88.9889 57.7464) (end 91.7702 57.7464) (width 1) (layer B.Cu) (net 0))
 (segment (start 88.9889 59.7464) (end 91.7702 59.7464) (width 1) (layer B.Cu) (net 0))
 (segment (start 88.9889 61.7464) (end 91.7702 61.7464) (width 1) (layer B.Cu) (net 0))
 (segment (start 88.9889 69.5589) (end 91.7702 69.5589) (width 1) (layer B.Cu) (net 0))
 (segment (start 88.9889 71.5589) (end 91.7702 71.5589) (width 1) (layer B.Cu) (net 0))
 (segment (start 88.9889 73.5589) (end 91.7702 73.5589) (width 1) (layer B.Cu) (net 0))
 (segment (start 88.9889 75.5589) (end 91.7702 75.5589) (width 1) (layer B.Cu) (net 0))
 (segment (start 88.9889 77.5589) (end 91.7702 77.5589) (width 1) (layer B.Cu) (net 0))
 (segment (start 88.9889 79.5589) (end 91.7702 79.5589) (width 1) (layer B.Cu) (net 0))
 (segment (start 88.9889 81.5589) (end 91.7702 81.5589) (width 1) (layer B.Cu) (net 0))
 (segment (start 88.9889 83.5589) (end 91.7702 83.5589) (width 1) (layer B.Cu) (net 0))
 (segment (start 88.9889 85.5589) (end 91.7702 85.5589) (width 1) (layer B.Cu) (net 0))
 (segment (start 88.9889 88.6089) (end 91.7702 88.6089) (width 1) (layer B.Cu) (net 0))
 (segment (start 88.9889 90.6089) (end 91.7702 90.6089) (width 1) (layer B.Cu) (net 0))
 (segment (start 88.9889 92.6089) (end 91.7702 92.6089) (width 1) (layer B.Cu) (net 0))
 (segment (start 88.9889 94.6089) (end 91.7702 94.6089) (width 1) (layer B.Cu) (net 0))
 (segment (start 88.9889 96.6089) (end 91.7702 96.6089) (width 1) (layer B.Cu) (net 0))
 (segment (start 88.9889 98.6089) (end 91.7702 98.6089) (width 1) (layer B.Cu) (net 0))
 (segment (start 88.9889 100.6089) (end 91.7702 100.6089) (width 1) (layer B.Cu) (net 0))
 (segment (start 88.9889 102.6089) (end 91.7702 102.6089) (width 1) (layer B.Cu) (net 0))
 (segment (start 88.9889 104.6089) (end 91.7702 104.6089) (width 1) (layer B.Cu) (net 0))
 (segment (start 88.9889 107.6589) (end 91.7702 107.6589) (width 1) (layer B.Cu) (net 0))
 (segment (start 88.9889 109.6589) (end 91.7702 109.6589) (width 1) (layer B.Cu) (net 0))
 (segment (start 88.9889 111.6589) (end 91.7702 111.6589) (width 1) (layer B.Cu) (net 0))
 (segment (start 88.9889 113.6589) (end 91.7702 113.6589) (width 1) (layer B.Cu) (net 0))
 (segment (start 88.9889 115.6589) (end 91.7702 115.6589) (width 1) (layer B.Cu) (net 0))
 (segment (start 88.9889 117.6589) (end 91.7702 117.6589) (width 1) (layer B.Cu) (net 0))
 (segment (start 88.9889 119.6589) (end 91.7702 119.6589) (width 1) (layer B.Cu) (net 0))
 (segment (start 88.9889 121.6589) (end 91.7702 121.6589) (width 1) (layer B.Cu) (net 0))
 (segment (start 88.9889 123.6589) (end 91.7702 123.6589) (width 1) (layer B.Cu) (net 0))
 (segment (start 88.9889 126.7089) (end 91.7702 126.7089) (width 1) (layer B.Cu) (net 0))
 (segment (start 88.9889 128.7089) (end 91.7702 128.7089) (width 1) (layer B.Cu) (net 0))
 (segment (start 88.9889 130.7089) (end 91.7702 130.7089) (width 1) (layer B.Cu) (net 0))
 (segment (start 88.9889 132.7089) (end 91.7702 132.7089) (width 1) (layer B.Cu) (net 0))
 (segment (start 88.9889 134.7089) (end 91.7702 134.7089) (width 1) (layer B.Cu) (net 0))
 (segment (start 88.9889 136.7089) (end 91.7702 136.7089) (width 1) (layer B.Cu) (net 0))
 (segment (start 88.9889 138.7089) (end 91.7702 138.7089) (width 1) (layer B.Cu) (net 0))
 (segment (start 88.9889 140.7089) (end 91.7702 140.7089) (width 1) (layer B.Cu) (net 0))
 (segment (start 88.9889 142.7089) (end 91.7702 142.7089) (width 1) (layer B.Cu) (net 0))
 (segment (start 88.9889 145.7589) (end 91.7702 145.7589) (width 1) (layer B.Cu) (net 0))
 (segment (start 88.9889 147.7589) (end 91.7702 147.7589) (width 1) (layer B.Cu) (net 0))
 (segment (start 88.9889 149.7589) (end 91.7702 149.7589) (width 1) (layer B.Cu) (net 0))
 (segment (start 88.9889 151.7589) (end 91.7702 151.7589) (width 1) (layer B.Cu) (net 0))
 (segment (start 88.9889 153.7589) (end 91.7702 153.7589) (width 1) (layer B.Cu) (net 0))
 (segment (start 88.9889 155.7589) (end 91.7702 155.7589) (width 1) (layer B.Cu) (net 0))
 (segment (start 88.9889 157.7589) (end 91.7702 157.7589) (width 1) (layer B.Cu) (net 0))
 (segment (start 88.9889 159.7589) (end 91.7702 159.7589) (width 1) (layer B.Cu) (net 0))
 (segment (start 88.9889 161.7589) (end 91.7702 161.7589) (width 1) (layer B.Cu) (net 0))
 (segment (start 91.7702 153.7589) (end 88.9889 153.7589) (width 1) (layer F.Cu) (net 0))
 (segment (start 91.7702 85.5589) (end 88.9889 85.5589) (width 1) (layer F.Cu) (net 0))
 (segment (start 91.7702 61.7464) (end 88.9889 61.7464) (width 1) (layer F.Cu) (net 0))
 (segment (start 91.7702 109.6589) (end 88.9889 109.6589) (width 1) (layer F.Cu) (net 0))
 (segment (start 91.7702 128.7089) (end 88.9889 128.7089) (width 1) (layer F.Cu) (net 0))
 (segment (start 91.7702 90.6089) (end 88.9889 90.6089) (width 1) (layer F.Cu) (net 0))
 (segment (start 91.7702 142.7089) (end 88.9889 142.7089) (width 1) (layer F.Cu) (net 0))
 (segment (start 91.7702 71.5589) (end 88.9889 71.5589) (width 1) (layer F.Cu) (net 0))
 (segment (start 91.7702 47.7464) (end 88.9889 47.7464) (width 1) (layer F.Cu) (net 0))
 (segment (start 91.7702 157.7589) (end 88.9889 157.7589) (width 1) (layer F.Cu) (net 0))
 (segment (start 91.7702 113.6589) (end 88.9889 113.6589) (width 1) (layer F.Cu) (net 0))
 (segment (start 91.7702 94.6089) (end 88.9889 94.6089) (width 1) (layer F.Cu) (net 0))
 (segment (start 91.7702 132.7089) (end 88.9889 132.7089) (width 1) (layer F.Cu) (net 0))
 (segment (start 91.7702 147.7589) (end 88.9889 147.7589) (width 1) (layer F.Cu) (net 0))
 (segment (start 91.7702 75.5589) (end 88.9889 75.5589) (width 1) (layer F.Cu) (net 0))
 (segment (start 91.7702 51.7464) (end 88.9889 51.7464) (width 1) (layer F.Cu) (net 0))
 (segment (start 91.7702 117.6589) (end 88.9889 117.6589) (width 1) (layer F.Cu) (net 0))
 (segment (start 91.7702 98.6089) (end 88.9889 98.6089) (width 1) (layer F.Cu) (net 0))
 (segment (start 91.7702 79.5589) (end 88.9889 79.5589) (width 1) (layer F.Cu) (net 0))
 (segment (start 91.7702 55.7464) (end 88.9889 55.7464) (width 1) (layer F.Cu) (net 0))
 (segment (start 91.7702 161.7589) (end 88.9889 161.7589) (width 1) (layer F.Cu) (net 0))
 (segment (start 91.7702 136.7089) (end 88.9889 136.7089) (width 1) (layer F.Cu) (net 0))
 (segment (start 91.7702 121.6589) (end 88.9889 121.6589) (width 1) (layer F.Cu) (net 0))
 (segment (start 91.7702 151.7589) (end 88.9889 151.7589) (width 1) (layer F.Cu) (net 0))
 (segment (start 91.7702 102.6089) (end 88.9889 102.6089) (width 1) (layer F.Cu) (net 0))
 (segment (start 91.7702 59.7464) (end 88.9889 59.7464) (width 1) (layer F.Cu) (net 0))
 (segment (start 91.7702 83.5589) (end 88.9889 83.5589) (width 1) (layer F.Cu) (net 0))
 (segment (start 91.7702 107.6589) (end 88.9889 107.6589) (width 1) (layer F.Cu) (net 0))
 (segment (start 91.7702 126.7089) (end 88.9889 126.7089) (width 1) (layer F.Cu) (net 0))
 (segment (start 91.7702 140.7089) (end 88.9889 140.7089) (width 1) (layer F.Cu) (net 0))
 (segment (start 91.7702 69.5589) (end 88.9889 69.5589) (width 1) (layer F.Cu) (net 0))
 (segment (start 91.7702 88.6089) (end 88.9889 88.6089) (width 1) (layer F.Cu) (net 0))
 (segment (start 91.7702 45.7464) (end 88.9889 45.7464) (width 1) (layer F.Cu) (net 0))
 (segment (start 91.7702 155.7589) (end 88.9889 155.7589) (width 1) (layer F.Cu) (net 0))
 (segment (start 91.7702 111.6589) (end 88.9889 111.6589) (width 1) (layer F.Cu) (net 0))
 (segment (start 91.7702 92.6089) (end 88.9889 92.6089) (width 1) (layer F.Cu) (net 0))
 (segment (start 91.7702 145.7589) (end 88.9889 145.7589) (width 1) (layer F.Cu) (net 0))
 (segment (start 91.7702 73.5589) (end 88.9889 73.5589) (width 1) (layer F.Cu) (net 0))
 (segment (start 91.7702 130.7089) (end 88.9889 130.7089) (width 1) (layer F.Cu) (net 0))
 (segment (start 91.7702 49.7464) (end 88.9889 49.7464) (width 1) (layer F.Cu) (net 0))
 (segment (start 91.7702 115.6589) (end 88.9889 115.6589) (width 1) (layer F.Cu) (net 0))
 (segment (start 91.7702 159.7589) (end 88.9889 159.7589) (width 1) (layer F.Cu) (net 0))
 (segment (start 91.7702 96.6089) (end 88.9889 96.6089) (width 1) (layer F.Cu) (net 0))
 (segment (start 91.7702 53.7464) (end 88.9889 53.7464) (width 1) (layer F.Cu) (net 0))
 (segment (start 91.7702 77.5589) (end 88.9889 77.5589) (width 1) (layer F.Cu) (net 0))
 (segment (start 91.7702 134.7089) (end 88.9889 134.7089) (width 1) (layer F.Cu) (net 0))
 (segment (start 91.7702 119.6589) (end 88.9889 119.6589) (width 1) (layer F.Cu) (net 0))
 (segment (start 91.7702 149.7589) (end 88.9889 149.7589) (width 1) (layer F.Cu) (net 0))
 (segment (start 91.7702 100.6089) (end 88.9889 100.6089) (width 1) (layer F.Cu) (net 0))
 (segment (start 91.7702 81.5589) (end 88.9889 81.5589) (width 1) (layer F.Cu) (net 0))
 (segment (start 91.7702 57.7464) (end 88.9889 57.7464) (width 1) (layer F.Cu) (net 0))
 (segment (start 91.7702 138.7089) (end 88.9889 138.7089) (width 1) (layer F.Cu) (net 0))
 (segment (start 91.7702 123.6589) (end 88.9889 123.6589) (width 1) (layer F.Cu) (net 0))
 (segment (start 91.7702 104.6089) (end 88.9889 104.6089) (width 1) (layer F.Cu) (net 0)))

